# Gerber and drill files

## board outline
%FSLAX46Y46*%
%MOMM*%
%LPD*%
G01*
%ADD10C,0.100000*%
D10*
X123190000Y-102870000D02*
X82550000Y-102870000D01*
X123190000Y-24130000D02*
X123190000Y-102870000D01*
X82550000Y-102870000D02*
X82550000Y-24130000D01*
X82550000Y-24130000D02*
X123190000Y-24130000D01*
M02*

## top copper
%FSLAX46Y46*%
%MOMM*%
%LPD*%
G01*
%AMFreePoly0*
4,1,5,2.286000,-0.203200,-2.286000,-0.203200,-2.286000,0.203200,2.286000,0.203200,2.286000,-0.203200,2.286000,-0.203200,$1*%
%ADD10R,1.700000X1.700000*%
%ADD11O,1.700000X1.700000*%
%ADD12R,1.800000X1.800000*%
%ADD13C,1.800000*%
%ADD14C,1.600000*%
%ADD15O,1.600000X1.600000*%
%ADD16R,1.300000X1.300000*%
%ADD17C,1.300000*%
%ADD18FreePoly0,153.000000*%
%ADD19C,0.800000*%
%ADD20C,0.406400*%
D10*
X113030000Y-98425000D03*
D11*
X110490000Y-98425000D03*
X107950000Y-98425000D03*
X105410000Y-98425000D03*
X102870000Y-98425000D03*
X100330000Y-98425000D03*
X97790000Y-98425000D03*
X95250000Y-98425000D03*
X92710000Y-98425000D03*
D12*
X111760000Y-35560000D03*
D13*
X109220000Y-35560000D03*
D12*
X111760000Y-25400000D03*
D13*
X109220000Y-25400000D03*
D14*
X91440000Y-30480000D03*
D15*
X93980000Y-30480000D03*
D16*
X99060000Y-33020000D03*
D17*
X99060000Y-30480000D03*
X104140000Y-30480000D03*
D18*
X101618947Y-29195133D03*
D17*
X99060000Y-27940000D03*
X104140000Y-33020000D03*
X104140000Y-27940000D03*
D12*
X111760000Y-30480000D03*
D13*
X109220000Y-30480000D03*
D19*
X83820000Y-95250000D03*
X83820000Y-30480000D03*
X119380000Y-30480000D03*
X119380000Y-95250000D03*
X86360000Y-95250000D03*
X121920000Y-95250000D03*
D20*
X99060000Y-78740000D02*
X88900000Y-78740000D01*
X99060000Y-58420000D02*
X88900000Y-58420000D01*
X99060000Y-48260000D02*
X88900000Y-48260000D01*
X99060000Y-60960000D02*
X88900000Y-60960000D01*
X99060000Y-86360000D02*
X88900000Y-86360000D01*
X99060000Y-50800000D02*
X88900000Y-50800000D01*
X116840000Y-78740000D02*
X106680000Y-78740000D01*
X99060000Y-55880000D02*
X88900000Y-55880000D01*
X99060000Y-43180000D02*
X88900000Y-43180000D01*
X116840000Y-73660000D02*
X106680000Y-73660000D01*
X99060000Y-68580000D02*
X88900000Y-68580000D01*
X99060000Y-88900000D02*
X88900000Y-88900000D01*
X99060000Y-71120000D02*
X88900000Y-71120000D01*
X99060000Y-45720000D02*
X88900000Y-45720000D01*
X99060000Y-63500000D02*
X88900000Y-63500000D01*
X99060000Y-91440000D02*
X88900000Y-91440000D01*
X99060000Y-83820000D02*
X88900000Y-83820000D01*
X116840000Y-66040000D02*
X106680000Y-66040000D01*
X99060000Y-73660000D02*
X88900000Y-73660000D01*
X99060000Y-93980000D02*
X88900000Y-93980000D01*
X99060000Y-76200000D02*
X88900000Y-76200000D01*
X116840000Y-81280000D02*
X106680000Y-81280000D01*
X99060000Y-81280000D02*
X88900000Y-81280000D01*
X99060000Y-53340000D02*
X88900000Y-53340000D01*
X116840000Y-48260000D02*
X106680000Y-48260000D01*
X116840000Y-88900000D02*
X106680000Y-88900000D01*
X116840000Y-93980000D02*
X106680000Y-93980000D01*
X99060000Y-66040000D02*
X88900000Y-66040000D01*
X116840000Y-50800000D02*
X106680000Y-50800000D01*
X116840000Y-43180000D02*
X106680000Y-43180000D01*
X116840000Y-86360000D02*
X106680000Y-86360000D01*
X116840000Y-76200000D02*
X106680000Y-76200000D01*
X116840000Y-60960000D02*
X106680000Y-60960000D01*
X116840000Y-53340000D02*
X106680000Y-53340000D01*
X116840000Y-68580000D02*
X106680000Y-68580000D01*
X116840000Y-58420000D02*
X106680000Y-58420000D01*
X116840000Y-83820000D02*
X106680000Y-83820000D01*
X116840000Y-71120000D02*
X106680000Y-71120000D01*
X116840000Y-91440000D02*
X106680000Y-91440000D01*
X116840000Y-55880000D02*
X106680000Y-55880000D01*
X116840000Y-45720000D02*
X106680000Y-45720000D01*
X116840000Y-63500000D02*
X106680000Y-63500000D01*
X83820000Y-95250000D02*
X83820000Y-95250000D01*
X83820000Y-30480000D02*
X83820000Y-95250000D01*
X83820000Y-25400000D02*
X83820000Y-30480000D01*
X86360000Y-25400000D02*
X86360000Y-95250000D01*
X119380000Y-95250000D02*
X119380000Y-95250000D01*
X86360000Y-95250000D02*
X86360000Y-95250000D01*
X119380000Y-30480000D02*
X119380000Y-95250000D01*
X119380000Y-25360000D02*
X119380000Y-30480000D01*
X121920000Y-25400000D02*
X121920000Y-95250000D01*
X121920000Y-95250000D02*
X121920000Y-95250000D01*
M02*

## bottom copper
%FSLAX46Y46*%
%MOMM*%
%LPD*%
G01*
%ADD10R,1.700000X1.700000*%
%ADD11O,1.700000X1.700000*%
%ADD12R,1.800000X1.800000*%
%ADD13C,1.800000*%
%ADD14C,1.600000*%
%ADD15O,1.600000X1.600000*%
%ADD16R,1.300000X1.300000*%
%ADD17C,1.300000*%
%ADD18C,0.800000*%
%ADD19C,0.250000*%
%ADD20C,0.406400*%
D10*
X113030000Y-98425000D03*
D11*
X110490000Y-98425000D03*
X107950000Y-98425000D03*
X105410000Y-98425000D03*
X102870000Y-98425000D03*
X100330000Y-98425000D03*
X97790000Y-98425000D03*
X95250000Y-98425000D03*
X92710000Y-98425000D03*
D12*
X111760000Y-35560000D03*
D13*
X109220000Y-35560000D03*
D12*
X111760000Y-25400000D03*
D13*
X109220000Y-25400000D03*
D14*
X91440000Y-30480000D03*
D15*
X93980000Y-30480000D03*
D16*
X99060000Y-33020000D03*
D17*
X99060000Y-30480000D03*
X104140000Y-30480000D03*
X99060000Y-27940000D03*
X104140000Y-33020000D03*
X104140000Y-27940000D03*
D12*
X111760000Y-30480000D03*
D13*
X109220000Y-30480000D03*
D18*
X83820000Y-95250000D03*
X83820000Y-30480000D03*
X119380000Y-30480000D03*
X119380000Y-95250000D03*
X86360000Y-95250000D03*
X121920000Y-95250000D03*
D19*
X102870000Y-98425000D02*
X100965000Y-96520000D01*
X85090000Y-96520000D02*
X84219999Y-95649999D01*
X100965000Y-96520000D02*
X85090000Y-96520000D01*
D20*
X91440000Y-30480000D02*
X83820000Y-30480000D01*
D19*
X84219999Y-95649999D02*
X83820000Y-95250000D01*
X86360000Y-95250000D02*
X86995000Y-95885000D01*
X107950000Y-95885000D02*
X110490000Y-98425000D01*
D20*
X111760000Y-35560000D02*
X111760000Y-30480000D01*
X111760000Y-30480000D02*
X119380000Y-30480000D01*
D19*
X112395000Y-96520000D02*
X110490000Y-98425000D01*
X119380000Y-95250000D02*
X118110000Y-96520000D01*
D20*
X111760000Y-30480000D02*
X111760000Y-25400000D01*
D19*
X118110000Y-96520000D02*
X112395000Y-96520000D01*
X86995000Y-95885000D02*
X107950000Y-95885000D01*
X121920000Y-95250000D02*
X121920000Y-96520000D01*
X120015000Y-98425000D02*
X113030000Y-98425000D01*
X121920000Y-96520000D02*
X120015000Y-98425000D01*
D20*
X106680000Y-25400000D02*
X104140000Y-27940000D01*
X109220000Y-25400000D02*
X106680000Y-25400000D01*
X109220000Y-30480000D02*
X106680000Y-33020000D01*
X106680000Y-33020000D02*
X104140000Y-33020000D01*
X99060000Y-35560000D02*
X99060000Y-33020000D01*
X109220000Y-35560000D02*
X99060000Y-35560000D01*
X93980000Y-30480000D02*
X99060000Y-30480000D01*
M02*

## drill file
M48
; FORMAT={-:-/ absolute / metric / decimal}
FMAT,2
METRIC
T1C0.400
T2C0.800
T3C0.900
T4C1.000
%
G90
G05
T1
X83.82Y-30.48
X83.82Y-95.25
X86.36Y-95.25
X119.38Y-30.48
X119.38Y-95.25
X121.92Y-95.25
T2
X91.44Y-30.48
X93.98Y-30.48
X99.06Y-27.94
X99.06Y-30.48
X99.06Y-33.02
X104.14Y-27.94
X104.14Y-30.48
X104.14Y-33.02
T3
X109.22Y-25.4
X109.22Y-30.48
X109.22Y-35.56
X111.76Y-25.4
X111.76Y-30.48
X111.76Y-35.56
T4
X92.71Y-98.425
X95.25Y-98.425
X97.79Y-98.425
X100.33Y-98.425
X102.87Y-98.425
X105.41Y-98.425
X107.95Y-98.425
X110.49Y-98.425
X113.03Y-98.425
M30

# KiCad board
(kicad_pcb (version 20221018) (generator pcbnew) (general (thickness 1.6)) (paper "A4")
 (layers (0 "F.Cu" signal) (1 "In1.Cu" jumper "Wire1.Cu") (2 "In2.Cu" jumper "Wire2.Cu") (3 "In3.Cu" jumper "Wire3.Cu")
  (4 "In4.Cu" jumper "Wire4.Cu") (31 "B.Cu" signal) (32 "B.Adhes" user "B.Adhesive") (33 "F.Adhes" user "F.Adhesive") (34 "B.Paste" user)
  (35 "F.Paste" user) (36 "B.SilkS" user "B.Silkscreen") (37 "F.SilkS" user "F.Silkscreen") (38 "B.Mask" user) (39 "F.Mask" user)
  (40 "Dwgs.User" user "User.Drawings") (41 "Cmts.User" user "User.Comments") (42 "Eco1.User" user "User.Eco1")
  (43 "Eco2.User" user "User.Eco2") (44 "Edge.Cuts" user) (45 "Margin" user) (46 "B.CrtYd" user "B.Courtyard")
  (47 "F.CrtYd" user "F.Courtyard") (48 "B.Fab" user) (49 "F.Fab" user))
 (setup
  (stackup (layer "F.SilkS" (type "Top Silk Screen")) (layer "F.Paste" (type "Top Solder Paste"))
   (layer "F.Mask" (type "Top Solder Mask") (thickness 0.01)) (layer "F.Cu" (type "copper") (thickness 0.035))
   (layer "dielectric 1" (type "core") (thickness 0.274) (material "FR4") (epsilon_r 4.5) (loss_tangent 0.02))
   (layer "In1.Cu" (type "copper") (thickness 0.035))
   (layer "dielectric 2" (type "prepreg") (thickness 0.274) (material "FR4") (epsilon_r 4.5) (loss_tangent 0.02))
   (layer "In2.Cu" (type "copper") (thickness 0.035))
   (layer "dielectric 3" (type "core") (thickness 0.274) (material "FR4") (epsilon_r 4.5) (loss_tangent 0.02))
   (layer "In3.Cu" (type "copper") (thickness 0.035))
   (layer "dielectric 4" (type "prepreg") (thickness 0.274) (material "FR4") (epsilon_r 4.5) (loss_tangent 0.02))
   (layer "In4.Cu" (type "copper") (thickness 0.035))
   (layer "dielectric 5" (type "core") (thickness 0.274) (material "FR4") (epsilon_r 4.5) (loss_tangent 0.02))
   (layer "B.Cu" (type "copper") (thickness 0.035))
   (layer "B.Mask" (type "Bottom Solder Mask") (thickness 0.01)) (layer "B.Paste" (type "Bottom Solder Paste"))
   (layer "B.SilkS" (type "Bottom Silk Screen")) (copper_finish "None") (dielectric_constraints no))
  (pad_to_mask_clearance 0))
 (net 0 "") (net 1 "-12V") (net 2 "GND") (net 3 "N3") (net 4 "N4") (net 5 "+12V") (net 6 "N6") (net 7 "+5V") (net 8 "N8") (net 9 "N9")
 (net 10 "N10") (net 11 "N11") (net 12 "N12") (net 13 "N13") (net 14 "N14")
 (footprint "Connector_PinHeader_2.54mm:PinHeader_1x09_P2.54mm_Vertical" (layer "F.Cu") (at 113.03 98.425 -90)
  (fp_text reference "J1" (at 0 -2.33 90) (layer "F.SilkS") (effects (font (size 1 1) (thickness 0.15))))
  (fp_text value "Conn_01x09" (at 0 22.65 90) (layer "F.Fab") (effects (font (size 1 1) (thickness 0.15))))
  (pad "1" thru_hole rect (at 0 0 270) (size 1.7 1.7) (drill 1) (layers "*.Cu" "*.Mask") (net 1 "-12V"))
  (pad "2" thru_hole oval (at 0 2.54 270) (size 1.7 1.7) (drill 1) (layers "*.Cu" "*.Mask") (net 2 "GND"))
  (pad "3" thru_hole oval (at 0 5.08 270) (size 1.7 1.7) (drill 1) (layers "*.Cu" "*.Mask") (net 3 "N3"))
  (pad "4" thru_hole oval (at 0 7.62 270) (size 1.7 1.7) (drill 1) (layers "*.Cu" "*.Mask") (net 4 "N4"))
  (pad "5" thru_hole oval (at 0 10.16 270) (size 1.7 1.7) (drill 1) (layers "*.Cu" "*.Mask") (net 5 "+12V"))
  (pad "6" thru_hole oval (at 0 12.7 270) (size 1.7 1.7) (drill 1) (layers "*.Cu" "*.Mask") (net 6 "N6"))
  (pad "7" thru_hole oval (at 0 15.24 270) (size 1.7 1.7) (drill 1) (layers "*.Cu" "*.Mask") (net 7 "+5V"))
  (pad "8" thru_hole oval (at 0 17.78 270) (size 1.7 1.7) (drill 1) (layers "*.Cu" "*.Mask") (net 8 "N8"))
  (pad "9" thru_hole oval (at 0 20.32 270) (size 1.7 1.7) (drill 1) (layers "*.Cu" "*.Mask") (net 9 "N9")))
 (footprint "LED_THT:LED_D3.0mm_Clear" (layer "F.Cu") (at 111.76 35.56 180)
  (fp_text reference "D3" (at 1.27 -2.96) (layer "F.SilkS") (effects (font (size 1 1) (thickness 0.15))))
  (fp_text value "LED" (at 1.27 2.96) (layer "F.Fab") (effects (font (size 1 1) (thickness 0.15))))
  (pad "1" thru_hole rect (at 0 0 180) (size 1.8 1.8) (drill 0.9) (layers "*.Cu" "*.Mask") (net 2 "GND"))
  (pad "2" thru_hole circle (at 2.54 0 180) (size 1.8 1.8) (drill 0.9) (layers "*.Cu" "*.Mask") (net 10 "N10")))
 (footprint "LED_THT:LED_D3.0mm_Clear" (layer "F.Cu") (at 111.76 25.4 180)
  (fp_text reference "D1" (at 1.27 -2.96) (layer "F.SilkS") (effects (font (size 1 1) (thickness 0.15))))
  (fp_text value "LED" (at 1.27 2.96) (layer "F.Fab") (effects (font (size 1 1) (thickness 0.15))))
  (pad "1" thru_hole rect (at 0 0 180) (size 1.8 1.8) (drill 0.9) (layers "*.Cu" "*.Mask") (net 2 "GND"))
  (pad "2" thru_hole circle (at 2.54 0 180) (size 1.8 1.8) (drill 0.9) (layers "*.Cu" "*.Mask") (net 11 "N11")))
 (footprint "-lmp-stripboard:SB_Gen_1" (layer "F.Cu") (at 91.44 30.48)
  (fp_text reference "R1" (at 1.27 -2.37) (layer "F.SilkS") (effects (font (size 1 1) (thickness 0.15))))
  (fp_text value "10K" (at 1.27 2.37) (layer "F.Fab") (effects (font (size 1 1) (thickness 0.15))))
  (pad "1" thru_hole circle (at 0 0) (size 1.6 1.6) (drill 0.8) (layers "*.Cu" "*.Mask") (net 5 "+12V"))
  (pad "2" thru_hole oval (at 2.54 0) (size 1.6 1.6) (drill 0.8) (layers "*.Cu" "*.Mask") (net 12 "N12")))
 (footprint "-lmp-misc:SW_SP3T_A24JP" (layer "F.Cu") (at 99.06 33.02 180)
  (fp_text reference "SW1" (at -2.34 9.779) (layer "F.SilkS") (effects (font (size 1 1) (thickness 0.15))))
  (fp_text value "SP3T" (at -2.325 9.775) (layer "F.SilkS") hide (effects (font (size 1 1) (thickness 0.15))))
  (pad "1" thru_hole rect (at 0 0 180) (size 1.3 1.3) (drill 0.8) (layers "*.Cu" "*.Mask") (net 10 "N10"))
  (pad "2" thru_hole circle (at 0 2.54 180) (size 1.3 1.3) (drill 0.8) (layers "*.Cu" "*.Mask") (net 12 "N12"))
  (pad "3" thru_hole circle (at -5.08 2.54 180) (size 1.3 1.3) (drill 0.8) (layers "*.Cu" "*.Mask") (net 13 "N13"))
  (pad "3" smd custom (at -2.1082 3.8354 153) (size 4.572 0.4064) (drill (offset -0.4064 0.19525)) (layers "F.Cu") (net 13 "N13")
   (options (clearance outline) (anchor rect)) (primitives))
  (pad "3" thru_hole circle (at 0 5.08 180) (size 1.3 1.3) (drill 0.8) (layers "*.Cu" "*.Mask") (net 13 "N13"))
  (pad "4" thru_hole circle (at -5.08 0 180) (size 1.3 1.3) (drill 0.8) (layers "*.Cu" "*.Mask") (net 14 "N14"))
  (pad "6" thru_hole circle (at -5.08 5.08 180) (size 1.3 1.3) (drill 0.8) (layers "*.Cu" "*.Mask") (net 11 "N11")))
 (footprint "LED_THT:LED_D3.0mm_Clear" (layer "F.Cu") (at 111.76 30.48 180)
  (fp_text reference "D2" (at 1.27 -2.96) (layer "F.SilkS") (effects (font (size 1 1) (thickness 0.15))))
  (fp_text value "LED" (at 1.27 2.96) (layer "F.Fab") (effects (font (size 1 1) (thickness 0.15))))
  (pad "1" thru_hole rect (at 0 0 180) (size 1.8 1.8) (drill 0.9) (layers "*.Cu" "*.Mask") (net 2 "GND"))
  (pad "2" thru_hole circle (at 2.54 0 180) (size 1.8 1.8) (drill 0.9) (layers "*.Cu" "*.Mask") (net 14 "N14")))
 (gr_line (start 123.19 102.87) (end 82.55 102.87) (stroke (width 0.1) (type solid)) (layer "Edge.Cuts"))
 (gr_line (start 123.19 24.13) (end 123.19 102.87) (stroke (width 0.1) (type solid)) (layer "Edge.Cuts"))
 (gr_line (start 82.55 102.87) (end 82.55 24.13) (stroke (width 0.1) (type solid)) (layer "Edge.Cuts"))
 (gr_line (start 82.55 24.13) (end 123.19 24.13) (stroke (width 0.1) (type solid)) (layer "Edge.Cuts"))
 (segment (start 99.06 78.74) (end 88.9 78.74) (width 0.4064) (layer "F.Cu") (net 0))
 (segment (start 99.06 58.42) (end 88.9 58.42) (width 0.4064) (layer "F.Cu") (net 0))
 (segment (start 99.06 48.26) (end 88.9 48.26) (width 0.4064) (layer "F.Cu") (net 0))
 (segment (start 99.06 60.96) (end 88.9 60.96) (width 0.4064) (layer "F.Cu") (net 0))
 (segment (start 99.06 86.36) (end 88.9 86.36) (width 0.4064) (layer "F.Cu") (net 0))
 (segment (start 99.06 50.8) (end 88.9 50.8) (width 0.4064) (layer "F.Cu") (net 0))
 (segment (start 116.84 78.74) (end 106.68 78.74) (width 0.4064) (layer "F.Cu") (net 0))
 (segment (start 99.06 55.88) (end 88.9 55.88) (width 0.4064) (layer "F.Cu") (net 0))
 (segment (start 99.06 43.18) (end 88.9 43.18) (width 0.4064) (layer "F.Cu") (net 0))
 (segment (start 116.84 73.66) (end 106.68 73.66) (width 0.4064) (layer "F.Cu") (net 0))
 (segment (start 99.06 68.58) (end 88.9 68.58) (width 0.4064) (layer "F.Cu") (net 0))
 (segment (start 99.06 88.9) (end 88.9 88.9) (width 0.4064) (layer "F.Cu") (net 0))
 (segment (start 99.06 71.12) (end 88.9 71.12) (width 0.4064) (layer "F.Cu") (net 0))
 (segment (start 99.06 45.72) (end 88.9 45.72) (width 0.4064) (layer "F.Cu") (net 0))
 (segment (start 99.06 63.5) (end 88.9 63.5) (width 0.4064) (layer "F.Cu") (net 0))
 (segment (start 99.06 91.44) (end 88.9 91.44) (width 0.4064) (layer "F.Cu") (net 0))
 (segment (start 99.06 83.82) (end 88.9 83.82) (width 0.4064) (layer "F.Cu") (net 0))
 (segment (start 116.84 66.04) (end 106.68 66.04) (width 0.4064) (layer "F.Cu") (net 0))
 (segment (start 99.06 73.66) (end 88.9 73.66) (width 0.4064) (layer "F.Cu") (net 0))
 (segment (start 99.06 93.98) (end 88.9 93.98) (width 0.4064) (layer "F.Cu") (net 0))
 (segment (start 99.06 76.2) (end 88.9 76.2) (width 0.4064) (layer "F.Cu") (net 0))
 (segment (start 116.84 81.28) (end 106.68 81.28) (width 0.4064) (layer "F.Cu") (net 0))
 (segment (start 99.06 81.28) (end 88.9 81.28) (width 0.4064) (layer "F.Cu") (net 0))
 (segment (start 99.06 53.34) (end 88.9 53.34) (width 0.4064) (layer "F.Cu") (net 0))
 (segment (start 116.84 48.26) (end 106.68 48.26) (width 0.4064) (layer "F.Cu") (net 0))
 (segment (start 116.84 88.9) (end 106.68 88.9) (width 0.4064) (layer "F.Cu") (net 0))
 (segment (start 116.84 93.98) (end 106.68 93.98) (width 0.4064) (layer "F.Cu") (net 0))
 (segment (start 99.06 66.04) (end 88.9 66.04) (width 0.4064) (layer "F.Cu") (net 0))
 (segment (start 116.84 50.8) (end 106.68 50.8) (width 0.4064) (layer "F.Cu") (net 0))
 (segment (start 116.84 43.18) (end 106.68 43.18) (width 0.4064) (layer "F.Cu") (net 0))
 (segment (start 116.84 86.36) (end 106.68 86.36) (width 0.4064) (layer "F.Cu") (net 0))
 (segment (start 116.84 76.2) (end 106.68 76.2) (width 0.4064) (layer "F.Cu") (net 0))
 (segment (start 116.84 60.96) (end 106.68 60.96) (width 0.4064) (layer "F.Cu") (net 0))
 (segment (start 116.84 53.34) (end 106.68 53.34) (width 0.4064) (layer "F.Cu") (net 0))
 (segment (start 116.84 68.58) (end 106.68 68.58) (width 0.4064) (layer "F.Cu") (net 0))
 (segment (start 116.84 58.42) (end 106.68 58.42) (width 0.4064) (layer "F.Cu") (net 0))
 (segment (start 116.84 83.82) (end 106.68 83.82) (width 0.4064) (layer "F.Cu") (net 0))
 (segment (start 116.84 71.12) (end 106.68 71.12) (width 0.4064) (layer "F.Cu") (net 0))
 (segment (start 116.84 91.44) (end 106.68 91.44) (width 0.4064) (layer "F.Cu") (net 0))
 (segment (start 116.84 55.88) (end 106.68 55.88) (width 0.4064) (layer "F.Cu") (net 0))
 (segment (start 116.84 45.72) (end 106.68 45.72) (width 0.4064) (layer "F.Cu") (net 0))
 (segment (start 116.84 63.5) (end 106.68 63.5) (width 0.4064) (layer "F.Cu") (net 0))
 (segment (start 83.82 95.25) (end 83.82 95.25) (width 0.4064) (layer "F.Cu") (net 5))
 (segment (start 83.82 30.48) (end 83.82 95.25) (width 0.4064) (layer "F.Cu") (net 5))
 (segment (start 83.82 25.4) (end 83.82 30.48) (width 0.4064) (layer "F.Cu") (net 5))
 (via (at 83.82 95.25) (size 0.8) (drill 0.4) (layers "F.Cu" "B.Cu") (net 5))
 (via (at 83.82 30.48) (size 0.8) (drill 0.4) (layers "F.Cu" "B.Cu") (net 5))
 (segment (start 102.87 98.425) (end 100.965 96.52) (width 0.25) (layer "B.Cu") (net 5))
 (segment (start 85.09 96.52) (end 84.219999 95.649999) (width 0.25) (layer "B.Cu") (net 5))
 (segment (start 100.965 96.52) (end 85.09 96.52) (width 0.25) (layer "B.Cu") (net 5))
 (segment (start 91.44 30.48) (end 83.82 30.48) (width 0.4064) (layer "B.Cu") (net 5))
 (segment (start 84.219999 95.649999) (end 83.82 95.25) (width 0.25) (layer "B.Cu") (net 5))
 (segment (start 86.36 25.4) (end 86.36 95.25) (width 0.4064) (layer "F.Cu") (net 2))
 (segment (start 119.38 95.25) (end 119.38 95.25) (width 0.4064) (layer "F.Cu") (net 2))
 (segment (start 86.36 95.25) (end 86.36 95.25) (width 0.4064) (layer "F.Cu") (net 2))
 (segment (start 119.38 30.48) (end 119.38 95.25) (width 0.4064) (layer "F.Cu") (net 2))
 (segment (start 119.38 25.36) (end 119.38 30.48) (width 0.4064) (layer "F.Cu") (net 2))
 (via (at 119.38 30.48) (size 0.8) (drill 0.4) (layers "F.Cu" "B.Cu") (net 2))
 (via (at 119.38 95.25) (size 0.8) (drill 0.4) (layers "F.Cu" "B.Cu") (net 2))
 (via (at 86.36 95.25) (size 0.8) (drill 0.4) (layers "F.Cu" "B.Cu") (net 2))
 (segment (start 86.36 95.25) (end 86.995 95.885) (width 0.25) (layer "B.Cu") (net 2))
 (segment (start 107.95 95.885) (end 110.49 98.425) (width 0.25) (layer "B.Cu") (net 2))
 (segment (start 111.76 35.56) (end 111.76 30.48) (width 0.4064) (layer "B.Cu") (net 2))
 (segment (start 111.76 30.48) (end 119.38 30.48) (width 0.4064) (layer "B.Cu") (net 2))
 (segment (start 112.395 96.52) (end 110.49 98.425) (width 0.25) (layer "B.Cu") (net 2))
 (segment (start 119.38 95.25) (end 118.11 96.52) (width 0.25) (layer "B.Cu") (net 2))
 (segment (start 111.76 30.48) (end 111.76 25.4) (width 0.4064) (layer "B.Cu") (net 2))
 (segment (start 118.11 96.52) (end 112.395 96.52) (width 0.25) (layer "B.Cu") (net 2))
 (segment (start 86.995 95.885) (end 107.95 95.885) (width 0.25) (layer "B.Cu") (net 2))
 (segment (start 121.92 25.4) (end 121.92 95.25) (width 0.4064) (layer "F.Cu") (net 1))
 (segment (start 121.92 95.25) (end 121.92 95.25) (width 0.4064) (layer "F.Cu") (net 1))
 (via (at 121.92 95.25) (size 0.8) (drill 0.4) (layers "F.Cu" "B.Cu") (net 1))
 (segment (start 121.92 95.25) (end 121.92 96.52) (width 0.25) (layer "B.Cu") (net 1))
 (segment (start 120.015 98.425) (end 113.03 98.425) (width 0.25) (layer "B.Cu") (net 1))
 (segment (start 121.92 96.52) (end 120.015 98.425) (width 0.25) (layer "B.Cu") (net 1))
 (segment (start 106.68 25.4) (end 104.14 27.94) (width 0.4064) (layer "B.Cu") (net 11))
 (segment (start 109.22 25.4) (end 106.68 25.4) (width 0.4064) (layer "B.Cu") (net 11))
 (segment (start 109.22 30.48) (end 106.68 33.02) (width 0.4064) (layer "B.Cu") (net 14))
 (segment (start 106.68 33.02) (end 104.14 33.02) (width 0.4064) (layer "B.Cu") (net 14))
 (segment (start 99.06 35.56) (end 99.06 33.02) (width 0.4064) (layer "B.Cu") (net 10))
 (segment (start 109.22 35.56) (end 99.06 35.56) (width 0.4064) (layer "B.Cu") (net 10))
 (segment (start 93.98 30.48) (end 99.06 30.48) (width 0.4064) (layer "B.Cu") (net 12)))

